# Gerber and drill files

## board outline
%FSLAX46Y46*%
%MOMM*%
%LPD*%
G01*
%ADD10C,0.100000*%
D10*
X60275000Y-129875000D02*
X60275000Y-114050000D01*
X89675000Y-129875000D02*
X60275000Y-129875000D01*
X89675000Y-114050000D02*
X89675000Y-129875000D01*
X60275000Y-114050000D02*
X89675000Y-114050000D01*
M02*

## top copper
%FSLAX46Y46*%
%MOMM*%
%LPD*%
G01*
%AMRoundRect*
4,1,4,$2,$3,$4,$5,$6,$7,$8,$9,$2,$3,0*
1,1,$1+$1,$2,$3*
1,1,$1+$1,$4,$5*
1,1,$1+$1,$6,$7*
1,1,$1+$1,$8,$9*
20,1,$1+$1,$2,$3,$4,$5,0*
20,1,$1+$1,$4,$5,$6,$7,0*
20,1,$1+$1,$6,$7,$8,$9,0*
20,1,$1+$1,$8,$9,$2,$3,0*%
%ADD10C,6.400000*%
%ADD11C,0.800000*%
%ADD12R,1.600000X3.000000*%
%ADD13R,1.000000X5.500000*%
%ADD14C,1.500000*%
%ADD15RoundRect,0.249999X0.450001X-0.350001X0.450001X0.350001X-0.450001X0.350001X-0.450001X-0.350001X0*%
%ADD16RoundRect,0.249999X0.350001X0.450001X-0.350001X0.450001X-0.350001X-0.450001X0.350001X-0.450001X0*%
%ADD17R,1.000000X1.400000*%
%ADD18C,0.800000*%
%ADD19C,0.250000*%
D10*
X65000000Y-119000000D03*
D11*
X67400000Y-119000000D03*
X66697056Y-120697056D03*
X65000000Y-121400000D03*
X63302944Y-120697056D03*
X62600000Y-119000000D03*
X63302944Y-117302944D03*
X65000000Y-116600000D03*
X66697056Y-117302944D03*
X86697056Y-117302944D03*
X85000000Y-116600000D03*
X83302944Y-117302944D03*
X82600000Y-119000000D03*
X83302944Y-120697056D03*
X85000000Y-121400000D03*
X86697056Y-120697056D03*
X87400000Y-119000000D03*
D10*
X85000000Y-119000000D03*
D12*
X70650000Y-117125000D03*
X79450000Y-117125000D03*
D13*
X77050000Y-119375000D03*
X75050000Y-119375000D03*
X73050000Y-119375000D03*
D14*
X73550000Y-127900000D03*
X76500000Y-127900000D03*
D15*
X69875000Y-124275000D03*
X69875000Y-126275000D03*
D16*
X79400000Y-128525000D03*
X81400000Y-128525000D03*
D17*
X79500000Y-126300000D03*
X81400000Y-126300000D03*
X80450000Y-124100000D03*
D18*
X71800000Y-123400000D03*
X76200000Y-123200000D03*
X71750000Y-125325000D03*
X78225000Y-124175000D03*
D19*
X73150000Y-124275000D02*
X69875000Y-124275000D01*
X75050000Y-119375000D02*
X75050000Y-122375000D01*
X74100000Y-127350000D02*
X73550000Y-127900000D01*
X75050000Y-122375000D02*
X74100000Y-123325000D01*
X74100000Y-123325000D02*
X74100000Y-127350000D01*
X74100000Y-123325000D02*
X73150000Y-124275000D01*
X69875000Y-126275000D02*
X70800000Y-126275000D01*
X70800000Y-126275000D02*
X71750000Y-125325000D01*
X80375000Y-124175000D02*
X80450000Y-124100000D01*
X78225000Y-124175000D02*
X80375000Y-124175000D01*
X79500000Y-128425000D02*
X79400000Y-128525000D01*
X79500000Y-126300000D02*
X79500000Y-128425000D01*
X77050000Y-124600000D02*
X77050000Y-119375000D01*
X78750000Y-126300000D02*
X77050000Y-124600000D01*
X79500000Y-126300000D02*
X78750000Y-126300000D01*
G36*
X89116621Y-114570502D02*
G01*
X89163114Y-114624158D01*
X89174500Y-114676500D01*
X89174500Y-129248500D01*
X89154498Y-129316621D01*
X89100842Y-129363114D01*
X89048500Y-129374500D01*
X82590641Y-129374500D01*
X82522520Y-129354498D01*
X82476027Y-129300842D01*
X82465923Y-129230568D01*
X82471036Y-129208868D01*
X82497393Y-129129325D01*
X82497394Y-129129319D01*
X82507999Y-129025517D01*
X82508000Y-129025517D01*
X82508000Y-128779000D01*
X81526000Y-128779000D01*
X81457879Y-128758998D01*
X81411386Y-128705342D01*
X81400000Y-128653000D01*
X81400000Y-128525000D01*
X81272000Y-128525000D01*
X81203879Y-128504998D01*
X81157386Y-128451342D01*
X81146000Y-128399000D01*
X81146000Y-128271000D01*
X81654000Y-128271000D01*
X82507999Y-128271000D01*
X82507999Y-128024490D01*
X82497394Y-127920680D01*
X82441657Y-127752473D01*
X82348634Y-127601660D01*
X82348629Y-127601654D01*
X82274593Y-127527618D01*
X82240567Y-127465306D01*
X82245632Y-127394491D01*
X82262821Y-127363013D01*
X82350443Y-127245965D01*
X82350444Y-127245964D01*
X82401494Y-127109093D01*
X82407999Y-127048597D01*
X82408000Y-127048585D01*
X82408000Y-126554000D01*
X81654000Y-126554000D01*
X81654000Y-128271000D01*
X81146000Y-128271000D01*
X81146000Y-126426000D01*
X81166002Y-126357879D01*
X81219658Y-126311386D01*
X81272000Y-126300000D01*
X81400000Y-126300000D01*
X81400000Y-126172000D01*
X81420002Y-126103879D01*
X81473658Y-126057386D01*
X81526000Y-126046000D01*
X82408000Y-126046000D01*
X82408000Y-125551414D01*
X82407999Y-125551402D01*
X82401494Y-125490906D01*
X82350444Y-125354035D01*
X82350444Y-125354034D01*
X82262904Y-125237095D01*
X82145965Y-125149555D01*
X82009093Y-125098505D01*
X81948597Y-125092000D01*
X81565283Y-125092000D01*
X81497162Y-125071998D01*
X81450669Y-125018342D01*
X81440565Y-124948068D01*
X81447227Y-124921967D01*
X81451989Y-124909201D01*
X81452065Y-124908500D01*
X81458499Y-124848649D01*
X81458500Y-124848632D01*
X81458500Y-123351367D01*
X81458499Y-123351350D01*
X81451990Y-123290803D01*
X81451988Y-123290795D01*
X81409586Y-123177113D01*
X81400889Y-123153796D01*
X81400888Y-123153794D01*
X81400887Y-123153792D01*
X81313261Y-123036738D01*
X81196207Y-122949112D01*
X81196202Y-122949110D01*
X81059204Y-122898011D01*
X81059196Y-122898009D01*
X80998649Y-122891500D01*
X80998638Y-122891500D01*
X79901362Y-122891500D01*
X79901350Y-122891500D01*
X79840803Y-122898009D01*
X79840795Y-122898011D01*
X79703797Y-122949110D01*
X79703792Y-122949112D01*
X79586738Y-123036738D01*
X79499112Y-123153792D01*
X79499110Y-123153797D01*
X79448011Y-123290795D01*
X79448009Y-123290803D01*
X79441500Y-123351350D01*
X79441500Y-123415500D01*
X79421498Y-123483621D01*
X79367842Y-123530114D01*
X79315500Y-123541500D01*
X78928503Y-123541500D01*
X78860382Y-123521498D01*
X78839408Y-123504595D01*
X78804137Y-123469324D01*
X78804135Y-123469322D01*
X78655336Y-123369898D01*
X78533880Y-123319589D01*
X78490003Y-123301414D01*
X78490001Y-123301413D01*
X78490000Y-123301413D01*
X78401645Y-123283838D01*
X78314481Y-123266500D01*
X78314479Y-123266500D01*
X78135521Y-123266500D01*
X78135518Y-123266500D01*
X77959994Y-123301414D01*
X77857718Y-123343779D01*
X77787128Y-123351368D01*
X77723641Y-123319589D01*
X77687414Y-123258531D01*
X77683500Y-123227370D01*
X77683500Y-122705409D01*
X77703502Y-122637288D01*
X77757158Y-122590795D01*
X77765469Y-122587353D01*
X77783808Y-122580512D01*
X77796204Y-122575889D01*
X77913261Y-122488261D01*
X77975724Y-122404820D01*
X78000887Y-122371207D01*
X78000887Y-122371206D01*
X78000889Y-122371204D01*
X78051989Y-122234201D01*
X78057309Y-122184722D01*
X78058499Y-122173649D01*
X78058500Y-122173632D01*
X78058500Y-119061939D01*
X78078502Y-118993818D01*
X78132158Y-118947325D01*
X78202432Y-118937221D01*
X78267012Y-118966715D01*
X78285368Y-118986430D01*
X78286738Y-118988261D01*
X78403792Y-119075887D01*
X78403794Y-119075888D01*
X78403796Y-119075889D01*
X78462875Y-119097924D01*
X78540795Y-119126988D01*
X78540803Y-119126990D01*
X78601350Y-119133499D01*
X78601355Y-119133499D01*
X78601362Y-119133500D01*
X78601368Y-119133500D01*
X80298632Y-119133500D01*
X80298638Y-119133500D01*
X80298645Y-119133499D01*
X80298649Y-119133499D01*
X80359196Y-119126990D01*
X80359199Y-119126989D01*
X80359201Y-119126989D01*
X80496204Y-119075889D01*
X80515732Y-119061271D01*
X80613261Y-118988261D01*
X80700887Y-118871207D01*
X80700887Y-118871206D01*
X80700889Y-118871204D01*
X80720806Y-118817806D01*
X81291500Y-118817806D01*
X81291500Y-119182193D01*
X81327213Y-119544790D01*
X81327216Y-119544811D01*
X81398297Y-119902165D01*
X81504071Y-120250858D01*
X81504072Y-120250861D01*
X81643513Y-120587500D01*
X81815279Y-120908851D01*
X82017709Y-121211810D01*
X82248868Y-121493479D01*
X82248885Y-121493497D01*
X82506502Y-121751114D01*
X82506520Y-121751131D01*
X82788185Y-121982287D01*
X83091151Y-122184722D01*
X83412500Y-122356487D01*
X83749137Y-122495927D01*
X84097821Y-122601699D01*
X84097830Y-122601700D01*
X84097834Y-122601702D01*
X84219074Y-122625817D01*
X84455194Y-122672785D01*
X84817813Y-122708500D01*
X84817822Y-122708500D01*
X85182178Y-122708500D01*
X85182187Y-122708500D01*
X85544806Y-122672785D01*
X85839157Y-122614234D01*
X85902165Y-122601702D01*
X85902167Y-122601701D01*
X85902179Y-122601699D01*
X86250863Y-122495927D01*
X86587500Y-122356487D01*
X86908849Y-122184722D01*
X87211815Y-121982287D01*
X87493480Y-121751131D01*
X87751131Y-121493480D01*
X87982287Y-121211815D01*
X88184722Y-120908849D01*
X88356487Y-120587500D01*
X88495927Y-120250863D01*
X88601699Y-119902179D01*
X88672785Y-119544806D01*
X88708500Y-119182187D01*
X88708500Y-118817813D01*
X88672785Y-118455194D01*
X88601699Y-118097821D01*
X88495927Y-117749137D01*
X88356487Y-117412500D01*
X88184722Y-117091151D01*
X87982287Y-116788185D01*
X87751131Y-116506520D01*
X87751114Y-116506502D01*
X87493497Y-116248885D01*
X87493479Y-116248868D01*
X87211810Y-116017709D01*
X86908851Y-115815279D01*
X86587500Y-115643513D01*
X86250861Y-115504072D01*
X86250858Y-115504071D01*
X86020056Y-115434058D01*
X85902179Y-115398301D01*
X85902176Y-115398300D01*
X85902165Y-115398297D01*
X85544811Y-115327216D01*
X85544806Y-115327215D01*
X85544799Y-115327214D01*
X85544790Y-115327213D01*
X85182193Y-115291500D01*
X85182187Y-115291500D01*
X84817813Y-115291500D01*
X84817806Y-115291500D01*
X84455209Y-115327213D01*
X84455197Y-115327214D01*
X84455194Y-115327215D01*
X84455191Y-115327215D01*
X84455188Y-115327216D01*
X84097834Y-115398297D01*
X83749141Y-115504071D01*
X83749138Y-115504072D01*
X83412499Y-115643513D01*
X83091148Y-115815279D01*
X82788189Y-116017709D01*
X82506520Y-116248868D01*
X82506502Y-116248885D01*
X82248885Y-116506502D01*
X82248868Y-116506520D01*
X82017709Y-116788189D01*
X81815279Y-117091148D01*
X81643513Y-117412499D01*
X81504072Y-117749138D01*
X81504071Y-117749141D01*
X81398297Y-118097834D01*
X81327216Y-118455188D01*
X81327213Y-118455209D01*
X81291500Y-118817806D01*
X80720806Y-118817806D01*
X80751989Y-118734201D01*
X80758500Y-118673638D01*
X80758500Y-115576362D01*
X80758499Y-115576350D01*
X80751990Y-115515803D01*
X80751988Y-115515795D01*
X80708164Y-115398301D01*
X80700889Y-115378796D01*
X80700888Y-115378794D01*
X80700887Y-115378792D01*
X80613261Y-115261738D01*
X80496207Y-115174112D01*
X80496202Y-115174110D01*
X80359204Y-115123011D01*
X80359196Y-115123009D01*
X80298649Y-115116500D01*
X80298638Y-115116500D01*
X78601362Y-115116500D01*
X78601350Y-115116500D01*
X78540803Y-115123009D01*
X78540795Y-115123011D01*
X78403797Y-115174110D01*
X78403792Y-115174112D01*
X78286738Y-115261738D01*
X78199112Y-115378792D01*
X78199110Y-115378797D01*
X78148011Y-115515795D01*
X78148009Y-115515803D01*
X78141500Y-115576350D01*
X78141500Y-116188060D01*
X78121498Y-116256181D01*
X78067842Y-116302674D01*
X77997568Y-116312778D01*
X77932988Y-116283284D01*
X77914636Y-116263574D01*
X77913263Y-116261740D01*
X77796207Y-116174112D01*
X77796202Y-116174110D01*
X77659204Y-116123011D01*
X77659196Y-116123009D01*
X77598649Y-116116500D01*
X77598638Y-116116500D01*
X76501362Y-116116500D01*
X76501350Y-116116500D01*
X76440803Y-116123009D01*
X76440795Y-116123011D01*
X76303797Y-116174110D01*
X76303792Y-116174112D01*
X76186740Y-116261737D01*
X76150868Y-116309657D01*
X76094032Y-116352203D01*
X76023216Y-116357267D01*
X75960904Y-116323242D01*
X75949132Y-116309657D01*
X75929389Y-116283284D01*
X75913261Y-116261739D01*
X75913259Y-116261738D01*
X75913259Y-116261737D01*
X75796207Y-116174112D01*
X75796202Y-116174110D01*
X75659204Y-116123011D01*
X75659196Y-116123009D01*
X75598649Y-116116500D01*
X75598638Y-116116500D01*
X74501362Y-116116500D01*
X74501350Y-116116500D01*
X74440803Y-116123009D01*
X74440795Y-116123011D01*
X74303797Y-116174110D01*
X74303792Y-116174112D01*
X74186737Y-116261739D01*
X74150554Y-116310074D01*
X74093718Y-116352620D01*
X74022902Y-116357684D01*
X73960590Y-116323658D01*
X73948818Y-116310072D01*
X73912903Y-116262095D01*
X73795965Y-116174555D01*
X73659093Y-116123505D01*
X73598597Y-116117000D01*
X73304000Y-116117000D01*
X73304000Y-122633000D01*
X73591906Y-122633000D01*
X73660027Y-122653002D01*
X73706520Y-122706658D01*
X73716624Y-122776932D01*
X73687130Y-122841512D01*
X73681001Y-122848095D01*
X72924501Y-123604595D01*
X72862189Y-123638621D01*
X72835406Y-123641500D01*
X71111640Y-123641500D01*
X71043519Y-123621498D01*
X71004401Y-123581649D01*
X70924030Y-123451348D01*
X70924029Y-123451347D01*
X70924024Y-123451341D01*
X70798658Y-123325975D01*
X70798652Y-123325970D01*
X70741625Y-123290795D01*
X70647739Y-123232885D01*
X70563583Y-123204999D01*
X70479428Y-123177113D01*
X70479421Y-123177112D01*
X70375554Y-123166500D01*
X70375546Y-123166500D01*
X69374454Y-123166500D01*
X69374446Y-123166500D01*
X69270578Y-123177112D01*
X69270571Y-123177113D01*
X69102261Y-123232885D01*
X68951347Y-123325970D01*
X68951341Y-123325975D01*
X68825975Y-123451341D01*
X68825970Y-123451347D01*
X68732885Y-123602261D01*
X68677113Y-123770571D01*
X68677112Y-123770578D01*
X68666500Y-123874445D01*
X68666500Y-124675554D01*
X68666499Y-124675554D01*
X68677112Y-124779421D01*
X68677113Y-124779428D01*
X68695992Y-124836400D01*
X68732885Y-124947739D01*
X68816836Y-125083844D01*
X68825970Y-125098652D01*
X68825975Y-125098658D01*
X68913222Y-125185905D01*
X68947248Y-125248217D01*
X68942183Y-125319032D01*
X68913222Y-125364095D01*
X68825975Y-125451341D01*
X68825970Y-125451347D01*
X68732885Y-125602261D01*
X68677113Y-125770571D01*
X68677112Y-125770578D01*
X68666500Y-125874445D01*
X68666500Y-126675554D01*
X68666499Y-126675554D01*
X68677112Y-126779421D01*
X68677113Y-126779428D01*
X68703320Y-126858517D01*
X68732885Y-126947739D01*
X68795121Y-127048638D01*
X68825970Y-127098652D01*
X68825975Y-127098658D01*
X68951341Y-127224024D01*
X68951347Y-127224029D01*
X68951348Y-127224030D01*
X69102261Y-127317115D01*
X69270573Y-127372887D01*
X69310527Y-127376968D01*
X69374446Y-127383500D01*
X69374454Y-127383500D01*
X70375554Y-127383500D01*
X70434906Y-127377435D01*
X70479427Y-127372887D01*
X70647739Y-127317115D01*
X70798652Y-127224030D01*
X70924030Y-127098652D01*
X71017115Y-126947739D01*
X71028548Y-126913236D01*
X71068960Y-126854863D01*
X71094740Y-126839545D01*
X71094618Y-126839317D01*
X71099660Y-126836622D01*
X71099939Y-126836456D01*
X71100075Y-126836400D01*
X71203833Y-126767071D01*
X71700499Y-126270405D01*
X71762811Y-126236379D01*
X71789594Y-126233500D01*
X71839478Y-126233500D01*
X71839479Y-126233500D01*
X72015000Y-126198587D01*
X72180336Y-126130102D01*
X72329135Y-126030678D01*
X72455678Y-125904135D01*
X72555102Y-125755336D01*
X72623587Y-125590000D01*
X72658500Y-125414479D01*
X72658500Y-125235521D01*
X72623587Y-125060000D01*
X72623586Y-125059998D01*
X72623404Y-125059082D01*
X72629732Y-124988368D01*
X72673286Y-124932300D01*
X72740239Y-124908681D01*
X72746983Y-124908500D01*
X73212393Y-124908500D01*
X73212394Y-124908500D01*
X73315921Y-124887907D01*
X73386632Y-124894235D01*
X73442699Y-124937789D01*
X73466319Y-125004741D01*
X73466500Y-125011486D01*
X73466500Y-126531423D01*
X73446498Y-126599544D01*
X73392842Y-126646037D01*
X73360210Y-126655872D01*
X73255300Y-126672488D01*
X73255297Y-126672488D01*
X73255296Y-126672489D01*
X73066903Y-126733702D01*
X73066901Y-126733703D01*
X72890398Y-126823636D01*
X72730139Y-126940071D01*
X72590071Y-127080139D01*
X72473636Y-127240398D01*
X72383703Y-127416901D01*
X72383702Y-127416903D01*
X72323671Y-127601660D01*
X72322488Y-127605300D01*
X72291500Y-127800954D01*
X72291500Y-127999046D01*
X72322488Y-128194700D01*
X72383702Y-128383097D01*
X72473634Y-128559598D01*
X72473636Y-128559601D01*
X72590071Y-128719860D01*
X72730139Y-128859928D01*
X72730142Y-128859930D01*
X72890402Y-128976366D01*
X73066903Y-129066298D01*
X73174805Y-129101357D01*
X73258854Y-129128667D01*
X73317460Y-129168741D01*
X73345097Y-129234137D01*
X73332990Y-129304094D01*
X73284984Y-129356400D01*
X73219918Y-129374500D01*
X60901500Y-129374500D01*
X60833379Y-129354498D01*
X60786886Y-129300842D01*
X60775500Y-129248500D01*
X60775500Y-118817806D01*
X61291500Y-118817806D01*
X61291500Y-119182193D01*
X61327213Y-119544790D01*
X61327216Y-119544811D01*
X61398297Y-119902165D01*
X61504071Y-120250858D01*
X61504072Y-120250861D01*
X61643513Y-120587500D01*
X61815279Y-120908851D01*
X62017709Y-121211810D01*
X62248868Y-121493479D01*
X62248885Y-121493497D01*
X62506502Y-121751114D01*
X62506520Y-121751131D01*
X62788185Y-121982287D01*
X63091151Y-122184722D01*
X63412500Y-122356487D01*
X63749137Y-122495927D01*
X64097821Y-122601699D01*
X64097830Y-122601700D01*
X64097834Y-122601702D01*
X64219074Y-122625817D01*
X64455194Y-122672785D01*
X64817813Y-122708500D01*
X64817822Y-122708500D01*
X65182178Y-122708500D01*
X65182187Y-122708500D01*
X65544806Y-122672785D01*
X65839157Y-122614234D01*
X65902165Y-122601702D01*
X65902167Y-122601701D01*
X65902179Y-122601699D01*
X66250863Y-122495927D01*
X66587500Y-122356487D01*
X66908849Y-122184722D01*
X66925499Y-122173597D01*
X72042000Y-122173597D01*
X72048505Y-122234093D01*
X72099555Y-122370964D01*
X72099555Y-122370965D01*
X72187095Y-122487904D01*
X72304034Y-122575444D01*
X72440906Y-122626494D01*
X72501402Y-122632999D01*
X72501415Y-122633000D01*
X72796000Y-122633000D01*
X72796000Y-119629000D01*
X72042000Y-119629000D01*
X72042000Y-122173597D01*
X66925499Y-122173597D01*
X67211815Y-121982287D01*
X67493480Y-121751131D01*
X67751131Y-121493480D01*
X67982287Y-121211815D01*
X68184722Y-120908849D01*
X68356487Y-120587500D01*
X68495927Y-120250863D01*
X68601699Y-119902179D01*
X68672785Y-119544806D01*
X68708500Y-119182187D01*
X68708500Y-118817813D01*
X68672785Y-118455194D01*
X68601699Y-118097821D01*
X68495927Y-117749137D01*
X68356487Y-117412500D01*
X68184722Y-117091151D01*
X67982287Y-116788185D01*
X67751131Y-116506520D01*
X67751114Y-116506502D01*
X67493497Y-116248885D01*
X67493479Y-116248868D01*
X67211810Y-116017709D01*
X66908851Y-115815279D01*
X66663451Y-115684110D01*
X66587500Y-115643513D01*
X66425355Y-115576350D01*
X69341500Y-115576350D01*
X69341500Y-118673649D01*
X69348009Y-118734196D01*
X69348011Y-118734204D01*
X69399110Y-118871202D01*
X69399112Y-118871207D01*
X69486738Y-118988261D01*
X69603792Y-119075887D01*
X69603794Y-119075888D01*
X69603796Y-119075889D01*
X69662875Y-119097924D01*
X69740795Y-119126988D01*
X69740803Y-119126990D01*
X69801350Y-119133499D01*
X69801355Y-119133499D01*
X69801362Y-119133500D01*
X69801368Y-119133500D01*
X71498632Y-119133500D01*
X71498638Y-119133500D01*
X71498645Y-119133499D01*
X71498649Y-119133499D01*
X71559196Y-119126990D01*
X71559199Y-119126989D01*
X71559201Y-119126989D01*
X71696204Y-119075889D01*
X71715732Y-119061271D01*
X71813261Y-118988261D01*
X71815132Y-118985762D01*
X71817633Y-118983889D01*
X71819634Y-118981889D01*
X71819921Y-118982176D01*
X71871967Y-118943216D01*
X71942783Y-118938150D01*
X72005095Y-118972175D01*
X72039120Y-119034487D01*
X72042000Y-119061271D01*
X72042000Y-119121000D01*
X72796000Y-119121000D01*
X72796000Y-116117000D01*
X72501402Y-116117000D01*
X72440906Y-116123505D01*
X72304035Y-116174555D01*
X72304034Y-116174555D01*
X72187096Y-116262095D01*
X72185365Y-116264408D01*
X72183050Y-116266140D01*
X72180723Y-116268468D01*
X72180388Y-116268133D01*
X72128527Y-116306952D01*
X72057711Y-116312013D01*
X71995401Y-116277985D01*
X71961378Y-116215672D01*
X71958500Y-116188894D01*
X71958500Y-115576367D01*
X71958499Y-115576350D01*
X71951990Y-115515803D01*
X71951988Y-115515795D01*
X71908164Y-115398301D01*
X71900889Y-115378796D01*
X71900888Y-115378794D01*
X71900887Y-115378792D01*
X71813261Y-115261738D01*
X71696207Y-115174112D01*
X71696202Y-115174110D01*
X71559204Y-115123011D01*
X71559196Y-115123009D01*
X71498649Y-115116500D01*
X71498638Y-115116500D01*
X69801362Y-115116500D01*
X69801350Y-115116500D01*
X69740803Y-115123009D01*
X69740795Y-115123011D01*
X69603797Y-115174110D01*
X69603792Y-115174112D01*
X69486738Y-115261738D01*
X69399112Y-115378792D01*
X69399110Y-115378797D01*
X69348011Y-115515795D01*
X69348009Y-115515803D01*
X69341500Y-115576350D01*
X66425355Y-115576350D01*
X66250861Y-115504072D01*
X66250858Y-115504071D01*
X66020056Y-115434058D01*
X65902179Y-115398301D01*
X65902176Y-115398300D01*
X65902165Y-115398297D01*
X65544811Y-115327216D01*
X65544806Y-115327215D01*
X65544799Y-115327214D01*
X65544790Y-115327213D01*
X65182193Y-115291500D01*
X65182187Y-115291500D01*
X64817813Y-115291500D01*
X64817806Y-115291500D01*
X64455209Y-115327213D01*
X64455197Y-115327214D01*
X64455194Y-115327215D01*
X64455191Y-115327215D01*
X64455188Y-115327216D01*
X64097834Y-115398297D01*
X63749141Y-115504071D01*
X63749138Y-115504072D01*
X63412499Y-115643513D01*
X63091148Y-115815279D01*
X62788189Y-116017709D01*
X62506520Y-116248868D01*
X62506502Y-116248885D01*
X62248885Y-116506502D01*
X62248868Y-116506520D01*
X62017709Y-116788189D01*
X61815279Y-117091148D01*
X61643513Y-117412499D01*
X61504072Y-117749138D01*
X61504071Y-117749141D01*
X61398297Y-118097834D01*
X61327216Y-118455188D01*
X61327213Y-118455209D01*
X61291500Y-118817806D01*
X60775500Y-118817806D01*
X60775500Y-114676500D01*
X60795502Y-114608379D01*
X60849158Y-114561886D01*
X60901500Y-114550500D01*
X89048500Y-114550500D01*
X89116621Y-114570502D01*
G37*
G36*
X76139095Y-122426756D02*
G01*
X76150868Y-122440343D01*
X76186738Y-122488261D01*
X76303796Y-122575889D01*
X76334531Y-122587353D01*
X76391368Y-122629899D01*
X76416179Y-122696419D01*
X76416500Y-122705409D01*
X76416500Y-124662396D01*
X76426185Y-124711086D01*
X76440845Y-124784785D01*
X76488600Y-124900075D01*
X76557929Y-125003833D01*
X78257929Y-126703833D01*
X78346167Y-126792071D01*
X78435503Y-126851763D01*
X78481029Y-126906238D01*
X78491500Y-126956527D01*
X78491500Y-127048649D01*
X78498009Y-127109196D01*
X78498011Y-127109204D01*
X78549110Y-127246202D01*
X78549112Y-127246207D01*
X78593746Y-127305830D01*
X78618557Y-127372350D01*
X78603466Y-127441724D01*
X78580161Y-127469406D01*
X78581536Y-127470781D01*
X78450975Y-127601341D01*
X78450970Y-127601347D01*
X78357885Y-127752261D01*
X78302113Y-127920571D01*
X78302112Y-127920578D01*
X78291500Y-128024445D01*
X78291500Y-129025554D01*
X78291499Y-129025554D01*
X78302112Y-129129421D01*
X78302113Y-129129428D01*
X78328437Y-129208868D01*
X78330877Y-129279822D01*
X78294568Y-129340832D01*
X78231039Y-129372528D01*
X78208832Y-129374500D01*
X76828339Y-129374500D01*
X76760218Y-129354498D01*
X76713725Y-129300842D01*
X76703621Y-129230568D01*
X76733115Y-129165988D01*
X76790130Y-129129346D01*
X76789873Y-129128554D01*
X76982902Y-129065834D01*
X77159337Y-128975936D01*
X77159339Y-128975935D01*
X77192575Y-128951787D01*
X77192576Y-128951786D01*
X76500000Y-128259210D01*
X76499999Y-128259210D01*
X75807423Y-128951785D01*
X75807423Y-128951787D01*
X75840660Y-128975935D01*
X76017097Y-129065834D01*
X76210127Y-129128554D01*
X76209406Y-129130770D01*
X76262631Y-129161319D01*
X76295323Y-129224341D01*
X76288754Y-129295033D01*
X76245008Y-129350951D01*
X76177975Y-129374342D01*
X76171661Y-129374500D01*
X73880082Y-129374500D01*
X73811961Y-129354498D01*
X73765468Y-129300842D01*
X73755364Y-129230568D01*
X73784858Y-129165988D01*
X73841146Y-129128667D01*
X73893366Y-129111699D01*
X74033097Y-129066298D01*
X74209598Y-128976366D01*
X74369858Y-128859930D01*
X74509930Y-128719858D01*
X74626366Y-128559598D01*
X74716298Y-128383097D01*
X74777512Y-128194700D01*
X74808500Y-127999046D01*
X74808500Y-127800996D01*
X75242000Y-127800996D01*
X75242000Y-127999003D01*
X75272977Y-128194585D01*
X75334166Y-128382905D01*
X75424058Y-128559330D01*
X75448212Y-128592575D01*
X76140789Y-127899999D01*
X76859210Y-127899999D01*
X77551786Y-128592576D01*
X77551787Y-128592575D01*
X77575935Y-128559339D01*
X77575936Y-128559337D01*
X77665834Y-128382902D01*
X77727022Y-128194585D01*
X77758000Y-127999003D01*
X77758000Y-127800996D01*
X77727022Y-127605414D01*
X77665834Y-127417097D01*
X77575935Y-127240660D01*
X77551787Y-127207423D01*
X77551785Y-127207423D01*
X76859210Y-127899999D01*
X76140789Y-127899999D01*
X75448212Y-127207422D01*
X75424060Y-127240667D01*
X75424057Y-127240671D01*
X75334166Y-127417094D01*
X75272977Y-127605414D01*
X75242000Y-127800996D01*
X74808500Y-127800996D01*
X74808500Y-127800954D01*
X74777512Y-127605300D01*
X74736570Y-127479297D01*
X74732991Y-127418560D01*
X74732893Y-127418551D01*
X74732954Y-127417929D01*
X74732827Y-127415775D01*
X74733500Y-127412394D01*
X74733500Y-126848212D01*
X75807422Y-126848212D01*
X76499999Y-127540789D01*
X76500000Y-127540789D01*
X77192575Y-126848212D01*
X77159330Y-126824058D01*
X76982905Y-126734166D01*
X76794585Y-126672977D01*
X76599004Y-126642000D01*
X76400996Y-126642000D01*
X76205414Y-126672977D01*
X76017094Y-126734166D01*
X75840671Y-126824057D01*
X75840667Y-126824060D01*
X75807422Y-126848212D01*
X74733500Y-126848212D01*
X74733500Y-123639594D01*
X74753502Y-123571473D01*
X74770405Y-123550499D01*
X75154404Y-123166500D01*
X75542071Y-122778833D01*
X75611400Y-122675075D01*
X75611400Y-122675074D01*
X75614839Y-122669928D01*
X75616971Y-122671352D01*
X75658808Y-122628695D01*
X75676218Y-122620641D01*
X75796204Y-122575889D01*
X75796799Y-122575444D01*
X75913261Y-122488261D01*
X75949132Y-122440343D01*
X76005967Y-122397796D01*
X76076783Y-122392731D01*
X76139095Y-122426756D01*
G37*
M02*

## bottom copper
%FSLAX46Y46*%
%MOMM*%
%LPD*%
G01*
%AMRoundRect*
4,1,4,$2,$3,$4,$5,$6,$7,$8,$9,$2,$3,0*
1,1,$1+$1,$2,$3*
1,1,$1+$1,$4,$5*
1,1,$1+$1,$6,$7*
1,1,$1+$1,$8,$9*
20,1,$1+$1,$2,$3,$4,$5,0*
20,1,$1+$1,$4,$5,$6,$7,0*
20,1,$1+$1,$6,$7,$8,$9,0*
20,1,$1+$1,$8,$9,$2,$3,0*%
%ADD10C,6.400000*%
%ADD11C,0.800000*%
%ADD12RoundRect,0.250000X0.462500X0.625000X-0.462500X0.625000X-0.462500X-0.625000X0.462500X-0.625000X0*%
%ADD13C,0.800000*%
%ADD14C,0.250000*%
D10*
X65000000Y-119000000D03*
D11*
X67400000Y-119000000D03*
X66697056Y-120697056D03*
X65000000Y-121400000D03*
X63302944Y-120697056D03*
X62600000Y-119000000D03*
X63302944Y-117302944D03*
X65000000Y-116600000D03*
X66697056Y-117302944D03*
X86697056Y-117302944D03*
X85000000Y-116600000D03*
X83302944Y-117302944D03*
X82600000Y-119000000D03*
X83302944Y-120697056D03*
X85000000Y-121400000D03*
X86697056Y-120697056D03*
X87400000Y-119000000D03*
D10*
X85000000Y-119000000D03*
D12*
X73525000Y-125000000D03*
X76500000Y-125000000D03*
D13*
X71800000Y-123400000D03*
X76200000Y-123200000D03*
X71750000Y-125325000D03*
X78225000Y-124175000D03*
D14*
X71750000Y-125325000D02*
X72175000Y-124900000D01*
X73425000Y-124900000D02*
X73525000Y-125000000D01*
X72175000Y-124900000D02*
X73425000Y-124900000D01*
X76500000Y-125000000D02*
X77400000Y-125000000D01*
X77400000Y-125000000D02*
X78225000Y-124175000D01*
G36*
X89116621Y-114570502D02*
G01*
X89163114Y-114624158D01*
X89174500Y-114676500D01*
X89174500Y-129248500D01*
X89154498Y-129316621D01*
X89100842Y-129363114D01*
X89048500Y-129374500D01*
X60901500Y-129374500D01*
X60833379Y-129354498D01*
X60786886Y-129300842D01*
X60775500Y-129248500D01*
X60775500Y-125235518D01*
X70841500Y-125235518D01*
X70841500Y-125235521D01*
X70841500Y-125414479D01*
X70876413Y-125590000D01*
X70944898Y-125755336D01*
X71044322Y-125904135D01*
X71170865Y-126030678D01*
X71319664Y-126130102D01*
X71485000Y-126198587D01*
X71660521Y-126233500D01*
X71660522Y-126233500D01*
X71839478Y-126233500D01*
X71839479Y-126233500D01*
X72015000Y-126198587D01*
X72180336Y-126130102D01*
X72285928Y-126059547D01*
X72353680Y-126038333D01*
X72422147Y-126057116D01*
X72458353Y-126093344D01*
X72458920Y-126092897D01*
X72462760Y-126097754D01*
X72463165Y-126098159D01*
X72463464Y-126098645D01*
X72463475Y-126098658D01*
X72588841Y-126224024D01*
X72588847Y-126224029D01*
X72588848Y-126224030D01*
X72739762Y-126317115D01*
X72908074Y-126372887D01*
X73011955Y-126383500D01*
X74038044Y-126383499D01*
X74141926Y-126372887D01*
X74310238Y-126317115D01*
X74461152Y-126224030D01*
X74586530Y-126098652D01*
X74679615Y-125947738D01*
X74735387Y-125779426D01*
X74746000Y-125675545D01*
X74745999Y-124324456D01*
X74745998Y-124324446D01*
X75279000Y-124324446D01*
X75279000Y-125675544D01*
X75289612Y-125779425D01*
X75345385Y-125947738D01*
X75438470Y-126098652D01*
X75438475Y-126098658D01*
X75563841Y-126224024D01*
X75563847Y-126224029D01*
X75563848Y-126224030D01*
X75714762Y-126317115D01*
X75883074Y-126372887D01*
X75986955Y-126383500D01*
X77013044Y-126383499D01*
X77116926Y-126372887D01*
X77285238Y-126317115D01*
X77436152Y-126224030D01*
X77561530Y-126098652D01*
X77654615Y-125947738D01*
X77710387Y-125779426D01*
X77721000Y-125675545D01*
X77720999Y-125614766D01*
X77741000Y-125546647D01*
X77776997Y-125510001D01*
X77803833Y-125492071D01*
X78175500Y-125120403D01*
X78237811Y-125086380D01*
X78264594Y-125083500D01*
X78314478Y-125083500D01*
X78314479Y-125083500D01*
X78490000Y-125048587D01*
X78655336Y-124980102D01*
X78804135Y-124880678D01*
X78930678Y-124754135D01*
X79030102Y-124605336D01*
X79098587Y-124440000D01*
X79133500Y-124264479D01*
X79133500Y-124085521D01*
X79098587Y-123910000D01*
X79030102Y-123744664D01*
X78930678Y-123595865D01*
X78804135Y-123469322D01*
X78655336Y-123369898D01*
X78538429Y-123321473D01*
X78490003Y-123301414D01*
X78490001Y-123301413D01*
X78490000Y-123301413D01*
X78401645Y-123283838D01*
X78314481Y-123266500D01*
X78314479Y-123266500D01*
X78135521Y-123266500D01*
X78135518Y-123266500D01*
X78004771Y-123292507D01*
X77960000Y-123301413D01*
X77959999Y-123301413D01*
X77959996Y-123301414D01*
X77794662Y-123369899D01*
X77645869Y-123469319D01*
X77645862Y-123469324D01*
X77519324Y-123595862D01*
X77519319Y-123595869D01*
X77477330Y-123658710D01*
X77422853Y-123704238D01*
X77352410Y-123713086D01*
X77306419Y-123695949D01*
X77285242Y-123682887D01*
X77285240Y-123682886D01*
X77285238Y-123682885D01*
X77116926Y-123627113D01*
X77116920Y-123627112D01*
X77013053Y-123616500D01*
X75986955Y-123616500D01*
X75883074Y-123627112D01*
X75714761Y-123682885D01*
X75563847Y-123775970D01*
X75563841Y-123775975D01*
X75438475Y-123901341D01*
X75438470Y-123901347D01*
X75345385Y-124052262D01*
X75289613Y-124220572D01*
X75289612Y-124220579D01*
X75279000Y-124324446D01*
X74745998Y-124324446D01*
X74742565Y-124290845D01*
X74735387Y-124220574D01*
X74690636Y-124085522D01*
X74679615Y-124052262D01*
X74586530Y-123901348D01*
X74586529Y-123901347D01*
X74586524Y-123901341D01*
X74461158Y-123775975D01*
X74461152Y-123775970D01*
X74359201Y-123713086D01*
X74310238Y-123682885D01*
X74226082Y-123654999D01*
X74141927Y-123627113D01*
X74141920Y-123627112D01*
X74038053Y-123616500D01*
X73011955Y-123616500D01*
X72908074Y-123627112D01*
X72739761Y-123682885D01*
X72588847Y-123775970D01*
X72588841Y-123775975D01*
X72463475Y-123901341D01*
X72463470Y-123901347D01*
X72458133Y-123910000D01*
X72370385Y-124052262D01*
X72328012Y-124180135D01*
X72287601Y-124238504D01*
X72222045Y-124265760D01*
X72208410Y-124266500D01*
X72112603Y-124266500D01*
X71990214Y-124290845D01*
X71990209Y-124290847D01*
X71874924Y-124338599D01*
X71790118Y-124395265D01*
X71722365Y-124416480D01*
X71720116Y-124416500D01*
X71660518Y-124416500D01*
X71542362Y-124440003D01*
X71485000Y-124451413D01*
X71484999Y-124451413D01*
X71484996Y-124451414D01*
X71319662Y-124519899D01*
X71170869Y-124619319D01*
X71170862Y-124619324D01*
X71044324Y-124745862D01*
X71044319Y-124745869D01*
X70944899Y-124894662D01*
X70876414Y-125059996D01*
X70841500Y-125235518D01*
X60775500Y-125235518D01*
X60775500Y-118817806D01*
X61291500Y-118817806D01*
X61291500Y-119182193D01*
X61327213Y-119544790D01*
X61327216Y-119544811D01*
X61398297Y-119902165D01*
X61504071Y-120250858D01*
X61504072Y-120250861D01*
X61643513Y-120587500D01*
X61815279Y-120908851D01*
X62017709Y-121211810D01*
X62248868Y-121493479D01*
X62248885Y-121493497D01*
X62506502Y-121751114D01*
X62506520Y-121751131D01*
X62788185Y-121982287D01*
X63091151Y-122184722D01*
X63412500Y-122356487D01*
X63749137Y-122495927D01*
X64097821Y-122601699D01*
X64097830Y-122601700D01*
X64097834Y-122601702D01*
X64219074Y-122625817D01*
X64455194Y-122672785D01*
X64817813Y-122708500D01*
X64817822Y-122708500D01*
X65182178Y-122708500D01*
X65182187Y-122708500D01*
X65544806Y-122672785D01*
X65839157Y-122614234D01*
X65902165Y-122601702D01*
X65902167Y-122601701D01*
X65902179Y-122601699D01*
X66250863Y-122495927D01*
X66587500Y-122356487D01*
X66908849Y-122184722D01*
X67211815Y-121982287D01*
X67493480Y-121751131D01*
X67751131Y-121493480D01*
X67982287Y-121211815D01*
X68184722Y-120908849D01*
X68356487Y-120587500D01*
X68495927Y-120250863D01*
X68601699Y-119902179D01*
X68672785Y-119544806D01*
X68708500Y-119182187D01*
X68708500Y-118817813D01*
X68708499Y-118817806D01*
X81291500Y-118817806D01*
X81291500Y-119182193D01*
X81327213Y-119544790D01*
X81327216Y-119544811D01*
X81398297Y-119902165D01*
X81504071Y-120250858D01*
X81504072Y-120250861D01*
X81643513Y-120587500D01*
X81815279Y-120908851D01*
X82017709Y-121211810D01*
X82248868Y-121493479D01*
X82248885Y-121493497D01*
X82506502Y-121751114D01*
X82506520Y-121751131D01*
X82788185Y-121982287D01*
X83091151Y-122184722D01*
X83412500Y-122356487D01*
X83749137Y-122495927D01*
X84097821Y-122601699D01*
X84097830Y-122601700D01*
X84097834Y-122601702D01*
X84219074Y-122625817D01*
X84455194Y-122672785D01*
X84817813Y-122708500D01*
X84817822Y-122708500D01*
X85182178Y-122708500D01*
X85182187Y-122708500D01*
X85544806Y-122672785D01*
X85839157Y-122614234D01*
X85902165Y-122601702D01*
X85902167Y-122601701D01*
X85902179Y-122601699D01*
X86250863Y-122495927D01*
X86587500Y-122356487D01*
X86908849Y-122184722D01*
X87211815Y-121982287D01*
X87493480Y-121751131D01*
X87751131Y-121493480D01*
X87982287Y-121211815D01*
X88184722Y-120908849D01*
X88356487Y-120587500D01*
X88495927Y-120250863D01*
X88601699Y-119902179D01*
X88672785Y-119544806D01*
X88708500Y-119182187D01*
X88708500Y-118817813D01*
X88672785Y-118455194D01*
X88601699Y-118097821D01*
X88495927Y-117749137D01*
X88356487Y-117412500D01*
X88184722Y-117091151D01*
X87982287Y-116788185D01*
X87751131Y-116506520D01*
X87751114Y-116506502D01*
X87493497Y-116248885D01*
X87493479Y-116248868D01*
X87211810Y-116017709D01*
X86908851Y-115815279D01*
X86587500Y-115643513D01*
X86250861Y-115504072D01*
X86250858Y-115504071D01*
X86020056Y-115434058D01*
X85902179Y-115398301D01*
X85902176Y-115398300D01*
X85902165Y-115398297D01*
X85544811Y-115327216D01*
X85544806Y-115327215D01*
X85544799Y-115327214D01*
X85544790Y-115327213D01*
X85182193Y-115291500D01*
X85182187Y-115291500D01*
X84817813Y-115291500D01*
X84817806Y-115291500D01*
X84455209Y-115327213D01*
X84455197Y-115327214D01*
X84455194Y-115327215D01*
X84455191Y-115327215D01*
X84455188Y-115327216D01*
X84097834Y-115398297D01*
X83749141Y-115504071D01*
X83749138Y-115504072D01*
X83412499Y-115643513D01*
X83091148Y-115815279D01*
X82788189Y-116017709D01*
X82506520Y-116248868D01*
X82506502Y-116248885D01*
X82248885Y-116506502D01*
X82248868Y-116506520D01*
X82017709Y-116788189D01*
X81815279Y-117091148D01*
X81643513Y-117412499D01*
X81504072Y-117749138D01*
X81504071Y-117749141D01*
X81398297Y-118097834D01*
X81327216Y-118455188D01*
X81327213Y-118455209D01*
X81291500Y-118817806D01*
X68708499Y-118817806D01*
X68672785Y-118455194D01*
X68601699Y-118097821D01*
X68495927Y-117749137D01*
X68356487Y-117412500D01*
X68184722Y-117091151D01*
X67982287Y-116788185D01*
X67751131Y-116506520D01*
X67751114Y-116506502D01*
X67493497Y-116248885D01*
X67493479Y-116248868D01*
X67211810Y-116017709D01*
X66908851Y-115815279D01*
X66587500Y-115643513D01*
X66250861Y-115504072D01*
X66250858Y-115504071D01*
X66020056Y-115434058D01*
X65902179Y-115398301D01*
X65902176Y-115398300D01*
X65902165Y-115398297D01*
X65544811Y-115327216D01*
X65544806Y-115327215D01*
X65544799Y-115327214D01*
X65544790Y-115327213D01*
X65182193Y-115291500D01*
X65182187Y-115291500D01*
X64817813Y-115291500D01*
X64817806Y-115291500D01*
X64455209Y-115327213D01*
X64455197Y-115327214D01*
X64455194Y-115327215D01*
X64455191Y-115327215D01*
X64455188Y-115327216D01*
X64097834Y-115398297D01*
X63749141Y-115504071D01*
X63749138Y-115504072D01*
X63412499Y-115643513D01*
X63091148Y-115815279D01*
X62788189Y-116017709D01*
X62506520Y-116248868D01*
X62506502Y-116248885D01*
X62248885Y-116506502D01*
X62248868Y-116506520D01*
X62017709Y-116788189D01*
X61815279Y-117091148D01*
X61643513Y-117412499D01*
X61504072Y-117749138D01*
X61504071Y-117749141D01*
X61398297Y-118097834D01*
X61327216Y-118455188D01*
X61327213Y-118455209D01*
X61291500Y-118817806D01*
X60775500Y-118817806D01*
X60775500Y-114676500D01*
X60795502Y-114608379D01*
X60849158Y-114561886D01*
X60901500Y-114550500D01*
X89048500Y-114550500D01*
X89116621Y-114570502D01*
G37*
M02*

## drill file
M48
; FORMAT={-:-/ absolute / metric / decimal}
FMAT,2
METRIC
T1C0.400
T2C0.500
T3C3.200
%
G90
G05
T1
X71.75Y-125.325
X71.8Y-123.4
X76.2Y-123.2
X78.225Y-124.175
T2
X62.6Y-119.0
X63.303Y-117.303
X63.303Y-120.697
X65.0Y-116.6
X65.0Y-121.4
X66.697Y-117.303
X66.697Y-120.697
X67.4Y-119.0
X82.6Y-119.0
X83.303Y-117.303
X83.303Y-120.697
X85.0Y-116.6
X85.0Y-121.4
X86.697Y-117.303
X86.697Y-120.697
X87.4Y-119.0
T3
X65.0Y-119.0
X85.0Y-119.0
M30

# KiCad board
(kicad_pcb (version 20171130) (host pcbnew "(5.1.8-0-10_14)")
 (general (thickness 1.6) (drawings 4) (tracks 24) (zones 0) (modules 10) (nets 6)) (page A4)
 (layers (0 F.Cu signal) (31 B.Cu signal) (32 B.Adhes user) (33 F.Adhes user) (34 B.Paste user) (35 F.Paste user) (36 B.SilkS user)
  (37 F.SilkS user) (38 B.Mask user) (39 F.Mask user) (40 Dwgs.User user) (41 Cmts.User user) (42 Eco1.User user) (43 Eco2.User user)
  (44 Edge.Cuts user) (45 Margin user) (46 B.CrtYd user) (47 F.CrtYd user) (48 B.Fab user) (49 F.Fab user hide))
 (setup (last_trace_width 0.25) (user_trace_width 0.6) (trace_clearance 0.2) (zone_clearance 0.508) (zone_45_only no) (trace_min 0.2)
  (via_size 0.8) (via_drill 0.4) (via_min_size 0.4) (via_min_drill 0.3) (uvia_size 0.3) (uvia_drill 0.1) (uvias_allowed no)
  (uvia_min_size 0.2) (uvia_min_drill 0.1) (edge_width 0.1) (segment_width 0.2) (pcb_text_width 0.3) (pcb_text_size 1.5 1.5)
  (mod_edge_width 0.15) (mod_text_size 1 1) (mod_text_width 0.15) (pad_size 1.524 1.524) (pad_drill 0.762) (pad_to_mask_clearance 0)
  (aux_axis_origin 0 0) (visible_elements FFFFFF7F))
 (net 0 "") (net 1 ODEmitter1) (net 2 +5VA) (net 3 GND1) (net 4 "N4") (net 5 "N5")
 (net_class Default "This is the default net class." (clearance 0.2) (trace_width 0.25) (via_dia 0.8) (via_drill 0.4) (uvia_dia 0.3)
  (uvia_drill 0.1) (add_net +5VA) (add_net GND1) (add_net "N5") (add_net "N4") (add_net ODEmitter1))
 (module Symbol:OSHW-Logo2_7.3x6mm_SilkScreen (layer F.Cu) (at 64.9 126.1)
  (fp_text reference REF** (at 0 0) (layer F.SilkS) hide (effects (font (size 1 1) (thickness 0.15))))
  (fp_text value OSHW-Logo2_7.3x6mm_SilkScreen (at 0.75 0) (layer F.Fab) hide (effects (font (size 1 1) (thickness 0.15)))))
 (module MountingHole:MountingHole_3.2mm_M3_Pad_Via (layer F.Cu) (at 65 119)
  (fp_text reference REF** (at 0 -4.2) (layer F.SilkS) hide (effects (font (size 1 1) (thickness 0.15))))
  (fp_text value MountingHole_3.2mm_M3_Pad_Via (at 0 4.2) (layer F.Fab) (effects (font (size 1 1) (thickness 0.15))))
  (pad 1 thru_hole circle (at 0 0) (size 6.4 6.4) (drill 3.2) (layers *.Cu *.Mask))
  (pad 1 thru_hole circle (at 2.4 0) (size 0.8 0.8) (drill 0.5) (layers *.Cu *.Mask))
  (pad 1 thru_hole circle (at 1.697056 1.697056) (size 0.8 0.8) (drill 0.5) (layers *.Cu *.Mask))
  (pad 1 thru_hole circle (at 0 2.4) (size 0.8 0.8) (drill 0.5) (layers *.Cu *.Mask))
  (pad 1 thru_hole circle (at -1.697056 1.697056) (size 0.8 0.8) (drill 0.5) (layers *.Cu *.Mask))
  (pad 1 thru_hole circle (at -2.4 0) (size 0.8 0.8) (drill 0.5) (layers *.Cu *.Mask))
  (pad 1 thru_hole circle (at -1.697056 -1.697056) (size 0.8 0.8) (drill 0.5) (layers *.Cu *.Mask))
  (pad 1 thru_hole circle (at 0 -2.4) (size 0.8 0.8) (drill 0.5) (layers *.Cu *.Mask))
  (pad 1 thru_hole circle (at 1.697056 -1.697056) (size 0.8 0.8) (drill 0.5) (layers *.Cu *.Mask)))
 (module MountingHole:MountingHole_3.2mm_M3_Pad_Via (layer F.Cu) (at 85 119)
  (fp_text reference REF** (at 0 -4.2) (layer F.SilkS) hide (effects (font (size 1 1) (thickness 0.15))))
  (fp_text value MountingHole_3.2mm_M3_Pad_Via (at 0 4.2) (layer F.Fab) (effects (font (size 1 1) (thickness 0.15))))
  (pad 1 thru_hole circle (at 1.697056 -1.697056) (size 0.8 0.8) (drill 0.5) (layers *.Cu *.Mask))
  (pad 1 thru_hole circle (at 0 -2.4) (size 0.8 0.8) (drill 0.5) (layers *.Cu *.Mask))
  (pad 1 thru_hole circle (at -1.697056 -1.697056) (size 0.8 0.8) (drill 0.5) (layers *.Cu *.Mask))
  (pad 1 thru_hole circle (at -2.4 0) (size 0.8 0.8) (drill 0.5) (layers *.Cu *.Mask))
  (pad 1 thru_hole circle (at -1.697056 1.697056) (size 0.8 0.8) (drill 0.5) (layers *.Cu *.Mask))
  (pad 1 thru_hole circle (at 0 2.4) (size 0.8 0.8) (drill 0.5) (layers *.Cu *.Mask))
  (pad 1 thru_hole circle (at 1.697056 1.697056) (size 0.8 0.8) (drill 0.5) (layers *.Cu *.Mask))
  (pad 1 thru_hole circle (at 2.4 0) (size 0.8 0.8) (drill 0.5) (layers *.Cu *.Mask))
  (pad 1 thru_hole circle (at 0 0) (size 6.4 6.4) (drill 3.2) (layers *.Cu *.Mask)))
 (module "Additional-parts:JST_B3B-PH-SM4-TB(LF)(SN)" (layer F.Cu) (at 75.05 117.125)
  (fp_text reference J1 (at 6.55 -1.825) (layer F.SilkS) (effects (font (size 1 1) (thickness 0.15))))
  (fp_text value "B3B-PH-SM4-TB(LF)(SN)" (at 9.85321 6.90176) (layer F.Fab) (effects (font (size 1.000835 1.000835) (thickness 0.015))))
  (pad 5 smd rect (at -4.4 0) (size 1.6 3) (layers F.Cu F.Paste F.Mask))
  (pad 4 smd rect (at 4.4 0) (size 1.6 3) (layers F.Cu F.Paste F.Mask))
  (pad 3 smd rect (at 2 2.25) (size 1 5.5) (layers F.Cu F.Paste F.Mask) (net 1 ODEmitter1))
  (pad 2 smd rect (at 0 2.25) (size 1 5.5) (layers F.Cu F.Paste F.Mask) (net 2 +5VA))
  (pad 1 smd rect (at -2 2.25) (size 1 5.5) (layers F.Cu F.Paste F.Mask) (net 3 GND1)))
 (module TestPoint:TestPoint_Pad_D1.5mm (layer F.Cu) (at 73.55 127.9)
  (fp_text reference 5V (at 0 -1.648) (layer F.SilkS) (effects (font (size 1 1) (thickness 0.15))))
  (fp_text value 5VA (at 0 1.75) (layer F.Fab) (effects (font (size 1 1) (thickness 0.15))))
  (pad 1 smd circle (at 0 0) (size 1.5 1.5) (layers F.Cu F.Mask) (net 2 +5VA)))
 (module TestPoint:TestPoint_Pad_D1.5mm (layer F.Cu) (at 76.5 127.9)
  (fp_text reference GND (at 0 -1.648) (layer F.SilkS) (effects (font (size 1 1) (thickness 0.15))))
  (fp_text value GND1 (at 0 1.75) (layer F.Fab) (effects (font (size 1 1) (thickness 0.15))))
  (pad 1 smd circle (at 0 0) (size 1.5 1.5) (layers F.Cu F.Mask) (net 3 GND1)))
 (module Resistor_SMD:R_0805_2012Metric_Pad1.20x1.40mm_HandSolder (layer F.Cu) (at 69.875 125.275 90)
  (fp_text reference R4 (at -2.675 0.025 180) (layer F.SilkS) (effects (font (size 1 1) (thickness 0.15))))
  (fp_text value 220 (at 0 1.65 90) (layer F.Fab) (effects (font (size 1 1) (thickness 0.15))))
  (pad 2 smd roundrect (at 1 0 90) (size 1.2 1.4) (layers F.Cu F.Paste F.Mask) (roundrect_rratio 0.2083325) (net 2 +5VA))
  (pad 1 smd roundrect (at -1 0 90) (size 1.2 1.4) (layers F.Cu F.Paste F.Mask) (roundrect_rratio 0.2083325) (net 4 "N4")))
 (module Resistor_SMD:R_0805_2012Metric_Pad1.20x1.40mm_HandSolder (layer F.Cu) (at 80.4 128.525 180)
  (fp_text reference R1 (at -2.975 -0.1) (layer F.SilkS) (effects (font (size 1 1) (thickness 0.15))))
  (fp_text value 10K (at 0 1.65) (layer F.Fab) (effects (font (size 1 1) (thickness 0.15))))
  (pad 2 smd roundrect (at 1 0 180) (size 1.2 1.4) (layers F.Cu F.Paste F.Mask) (roundrect_rratio 0.2083325) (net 1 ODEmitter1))
  (pad 1 smd roundrect (at -1 0 180) (size 1.2 1.4) (layers F.Cu F.Paste F.Mask) (roundrect_rratio 0.2083325) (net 3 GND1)))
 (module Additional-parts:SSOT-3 (layer F.Cu) (at 80.45 125.2)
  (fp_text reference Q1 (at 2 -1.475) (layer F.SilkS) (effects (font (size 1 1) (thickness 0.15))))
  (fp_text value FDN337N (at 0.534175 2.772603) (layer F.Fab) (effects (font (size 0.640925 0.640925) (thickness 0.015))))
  (pad 1 smd rect (at -0.95 1.1) (size 1 1.4) (layers F.Cu F.Paste F.Mask) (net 1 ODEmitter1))
  (pad 2 smd rect (at 0.95 1.1) (size 1 1.4) (layers F.Cu F.Paste F.Mask) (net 3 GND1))
  (pad 3 smd rect (at 0 -1.1) (size 1 1.4) (layers F.Cu F.Paste F.Mask) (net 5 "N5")))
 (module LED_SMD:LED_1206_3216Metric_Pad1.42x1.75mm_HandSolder (layer B.Cu) (at 75.0125 125 180)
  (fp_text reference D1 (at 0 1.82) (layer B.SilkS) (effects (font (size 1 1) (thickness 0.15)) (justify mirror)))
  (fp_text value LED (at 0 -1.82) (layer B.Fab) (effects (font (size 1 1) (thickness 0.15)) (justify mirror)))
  (pad 2 smd roundrect (at 1.4875 0 180) (size 1.425 1.75) (layers B.Cu B.Paste B.Mask) (roundrect_rratio 0.1754385964912281) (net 4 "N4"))
  (pad 1 smd roundrect (at -1.4875 0 180) (size 1.425 1.75) (layers B.Cu B.Paste B.Mask) (roundrect_rratio 0.1754385964912281) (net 5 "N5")))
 (gr_line (start 60.275 129.875) (end 60.275 114.05) (layer Edge.Cuts) (width 0.1))
 (gr_line (start 89.675 129.875) (end 60.275 129.875) (layer Edge.Cuts) (width 0.1))
 (gr_line (start 89.675 114.05) (end 89.675 129.875) (layer Edge.Cuts) (width 0.1))
 (gr_line (start 60.275 114.05) (end 89.675 114.05) (layer Edge.Cuts) (width 0.1))
 (via (at 71.8 123.4) (size 0.8) (drill 0.4) (layers F.Cu B.Cu) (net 3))
 (via (at 76.2 123.2) (size 0.8) (drill 0.4) (layers F.Cu B.Cu) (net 3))
 (segment (start 73.15 124.275) (end 69.875 124.275) (width 0.25) (layer F.Cu) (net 2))
 (segment (start 75.05 119.375) (end 75.05 122.375) (width 0.25) (layer F.Cu) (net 2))
 (segment (start 74.1 127.35) (end 73.55 127.9) (width 0.25) (layer F.Cu) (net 2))
 (segment (start 75.05 122.375) (end 74.1 123.325) (width 0.25) (layer F.Cu) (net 2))
 (segment (start 74.1 123.325) (end 74.1 127.35) (width 0.25) (layer F.Cu) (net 2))
 (segment (start 74.1 123.325) (end 73.15 124.275) (width 0.25) (layer F.Cu) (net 2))
 (segment (start 69.875 126.275) (end 70.8 126.275) (width 0.25) (layer F.Cu) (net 4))
 (via (at 71.75 125.325) (size 0.8) (drill 0.4) (layers F.Cu B.Cu) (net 4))
 (segment (start 70.8 126.275) (end 71.75 125.325) (width 0.25) (layer F.Cu) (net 4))
 (segment (start 71.75 125.325) (end 72.175 124.9) (width 0.25) (layer B.Cu) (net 4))
 (segment (start 73.425 124.9) (end 73.525 125) (width 0.25) (layer B.Cu) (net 4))
 (segment (start 72.175 124.9) (end 73.425 124.9) (width 0.25) (layer B.Cu) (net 4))
 (segment (start 76.5 125) (end 77.4 125) (width 0.25) (layer B.Cu) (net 5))
 (via (at 78.225 124.175) (size 0.8) (drill 0.4) (layers F.Cu B.Cu) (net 5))
 (segment (start 77.4 125) (end 78.225 124.175) (width 0.25) (layer B.Cu) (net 5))
 (segment (start 80.375 124.175) (end 80.45 124.1) (width 0.25) (layer F.Cu) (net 5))
 (segment (start 78.225 124.175) (end 80.375 124.175) (width 0.25) (layer F.Cu) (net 5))
 (segment (start 79.5 128.425) (end 79.4 128.525) (width 0.25) (layer F.Cu) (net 1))
 (segment (start 79.5 126.3) (end 79.5 128.425) (width 0.25) (layer F.Cu) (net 1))
 (segment (start 77.05 124.6) (end 77.05 119.375) (width 0.25) (layer F.Cu) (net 1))
 (segment (start 78.75 126.3) (end 77.05 124.6) (width 0.25) (layer F.Cu) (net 1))
 (segment (start 79.5 126.3) (end 78.75 126.3) (width 0.25) (layer F.Cu) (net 1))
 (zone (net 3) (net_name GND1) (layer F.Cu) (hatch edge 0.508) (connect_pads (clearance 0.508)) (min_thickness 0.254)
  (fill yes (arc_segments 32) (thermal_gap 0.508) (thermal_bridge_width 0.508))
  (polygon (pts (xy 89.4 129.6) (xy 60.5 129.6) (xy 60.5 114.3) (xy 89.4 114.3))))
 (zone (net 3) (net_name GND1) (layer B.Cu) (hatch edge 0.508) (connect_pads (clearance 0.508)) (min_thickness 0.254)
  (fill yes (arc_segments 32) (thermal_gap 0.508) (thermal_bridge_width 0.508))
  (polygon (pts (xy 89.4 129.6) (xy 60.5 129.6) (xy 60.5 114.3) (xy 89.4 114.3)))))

